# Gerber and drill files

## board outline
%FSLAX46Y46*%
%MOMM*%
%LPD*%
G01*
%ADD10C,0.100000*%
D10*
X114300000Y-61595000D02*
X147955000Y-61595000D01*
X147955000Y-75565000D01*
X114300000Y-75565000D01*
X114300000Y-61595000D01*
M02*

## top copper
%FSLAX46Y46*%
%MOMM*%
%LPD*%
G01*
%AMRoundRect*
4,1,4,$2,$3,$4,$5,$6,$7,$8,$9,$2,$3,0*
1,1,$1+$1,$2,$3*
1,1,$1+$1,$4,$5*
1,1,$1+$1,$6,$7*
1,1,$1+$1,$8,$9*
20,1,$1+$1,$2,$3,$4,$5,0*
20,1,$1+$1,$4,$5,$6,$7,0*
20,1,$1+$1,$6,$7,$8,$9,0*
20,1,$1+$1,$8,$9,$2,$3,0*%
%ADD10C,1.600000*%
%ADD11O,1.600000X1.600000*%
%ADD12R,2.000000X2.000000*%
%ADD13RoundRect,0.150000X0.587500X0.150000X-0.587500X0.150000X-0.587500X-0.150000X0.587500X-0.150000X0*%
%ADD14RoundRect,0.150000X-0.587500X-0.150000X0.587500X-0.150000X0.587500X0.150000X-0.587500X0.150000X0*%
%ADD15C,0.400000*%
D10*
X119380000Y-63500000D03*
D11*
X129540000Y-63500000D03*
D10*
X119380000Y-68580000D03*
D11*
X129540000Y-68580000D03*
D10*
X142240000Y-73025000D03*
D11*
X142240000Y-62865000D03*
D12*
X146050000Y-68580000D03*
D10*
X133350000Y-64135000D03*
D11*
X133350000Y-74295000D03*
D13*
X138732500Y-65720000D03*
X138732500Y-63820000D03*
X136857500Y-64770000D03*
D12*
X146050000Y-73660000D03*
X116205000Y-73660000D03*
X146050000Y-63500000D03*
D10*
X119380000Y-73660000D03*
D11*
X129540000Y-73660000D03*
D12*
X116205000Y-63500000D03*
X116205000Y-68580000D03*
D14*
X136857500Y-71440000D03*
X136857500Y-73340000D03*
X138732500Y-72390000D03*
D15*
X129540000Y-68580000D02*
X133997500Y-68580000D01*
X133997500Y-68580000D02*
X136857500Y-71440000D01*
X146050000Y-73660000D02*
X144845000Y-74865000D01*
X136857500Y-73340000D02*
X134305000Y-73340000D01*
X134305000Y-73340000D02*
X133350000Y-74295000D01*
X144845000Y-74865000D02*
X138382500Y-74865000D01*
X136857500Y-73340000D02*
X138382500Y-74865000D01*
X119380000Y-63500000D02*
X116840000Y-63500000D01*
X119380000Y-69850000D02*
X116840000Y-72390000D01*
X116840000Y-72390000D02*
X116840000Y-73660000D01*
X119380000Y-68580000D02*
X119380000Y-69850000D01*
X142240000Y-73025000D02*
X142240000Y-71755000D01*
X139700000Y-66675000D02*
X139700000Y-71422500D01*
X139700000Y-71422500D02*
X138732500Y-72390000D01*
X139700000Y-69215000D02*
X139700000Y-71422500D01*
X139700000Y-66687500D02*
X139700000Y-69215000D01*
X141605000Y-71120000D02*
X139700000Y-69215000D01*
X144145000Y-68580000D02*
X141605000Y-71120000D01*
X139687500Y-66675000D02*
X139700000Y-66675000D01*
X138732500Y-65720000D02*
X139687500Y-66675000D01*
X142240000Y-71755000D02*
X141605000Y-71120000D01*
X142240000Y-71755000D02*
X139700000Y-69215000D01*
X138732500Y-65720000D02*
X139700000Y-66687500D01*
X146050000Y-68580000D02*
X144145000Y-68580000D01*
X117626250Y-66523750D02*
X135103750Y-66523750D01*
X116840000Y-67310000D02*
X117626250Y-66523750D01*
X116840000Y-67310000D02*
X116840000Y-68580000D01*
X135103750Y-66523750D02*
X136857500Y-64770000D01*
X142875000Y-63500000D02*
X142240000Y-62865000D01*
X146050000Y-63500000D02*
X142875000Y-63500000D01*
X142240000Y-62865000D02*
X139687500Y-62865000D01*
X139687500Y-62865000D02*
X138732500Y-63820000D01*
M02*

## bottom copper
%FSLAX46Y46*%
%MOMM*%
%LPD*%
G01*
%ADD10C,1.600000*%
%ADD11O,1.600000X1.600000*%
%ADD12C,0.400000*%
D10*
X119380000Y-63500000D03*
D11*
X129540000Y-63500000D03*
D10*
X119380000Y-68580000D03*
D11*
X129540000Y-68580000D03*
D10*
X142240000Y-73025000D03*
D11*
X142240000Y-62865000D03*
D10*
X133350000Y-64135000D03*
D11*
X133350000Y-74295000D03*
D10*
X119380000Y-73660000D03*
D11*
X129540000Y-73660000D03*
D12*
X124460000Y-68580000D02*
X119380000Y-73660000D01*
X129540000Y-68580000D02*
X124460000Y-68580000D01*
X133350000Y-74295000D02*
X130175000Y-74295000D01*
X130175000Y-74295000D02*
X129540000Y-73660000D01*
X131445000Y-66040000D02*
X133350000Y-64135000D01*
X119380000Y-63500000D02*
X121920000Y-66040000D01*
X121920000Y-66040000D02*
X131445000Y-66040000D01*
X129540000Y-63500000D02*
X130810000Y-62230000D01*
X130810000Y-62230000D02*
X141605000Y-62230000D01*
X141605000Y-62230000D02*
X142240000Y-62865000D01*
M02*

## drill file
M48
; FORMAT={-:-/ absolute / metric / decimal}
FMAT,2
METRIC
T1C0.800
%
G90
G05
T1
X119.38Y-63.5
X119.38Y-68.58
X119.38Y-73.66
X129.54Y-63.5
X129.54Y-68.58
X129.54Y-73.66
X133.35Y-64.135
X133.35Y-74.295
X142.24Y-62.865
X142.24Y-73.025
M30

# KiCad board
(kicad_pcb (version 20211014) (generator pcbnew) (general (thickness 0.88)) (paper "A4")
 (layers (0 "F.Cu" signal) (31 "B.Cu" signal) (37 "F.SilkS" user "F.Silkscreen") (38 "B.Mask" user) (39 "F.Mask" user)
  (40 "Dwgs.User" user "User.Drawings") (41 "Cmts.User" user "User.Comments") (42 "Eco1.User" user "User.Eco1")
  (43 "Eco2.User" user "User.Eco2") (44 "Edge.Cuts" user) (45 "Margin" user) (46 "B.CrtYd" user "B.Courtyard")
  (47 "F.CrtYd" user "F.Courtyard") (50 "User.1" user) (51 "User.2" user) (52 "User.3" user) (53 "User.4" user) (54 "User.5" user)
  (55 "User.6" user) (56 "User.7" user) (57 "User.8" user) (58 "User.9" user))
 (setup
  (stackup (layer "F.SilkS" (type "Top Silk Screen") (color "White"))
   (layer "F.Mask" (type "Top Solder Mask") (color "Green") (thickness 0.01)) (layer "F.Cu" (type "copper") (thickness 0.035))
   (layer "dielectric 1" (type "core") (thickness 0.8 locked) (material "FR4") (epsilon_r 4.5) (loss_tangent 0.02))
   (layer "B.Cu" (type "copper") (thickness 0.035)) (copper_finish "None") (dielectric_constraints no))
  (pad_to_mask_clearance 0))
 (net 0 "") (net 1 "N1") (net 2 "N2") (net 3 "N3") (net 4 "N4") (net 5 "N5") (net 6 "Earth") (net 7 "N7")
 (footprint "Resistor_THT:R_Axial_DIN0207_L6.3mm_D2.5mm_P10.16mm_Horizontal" (layer "F.Cu") (at 119.38 63.5)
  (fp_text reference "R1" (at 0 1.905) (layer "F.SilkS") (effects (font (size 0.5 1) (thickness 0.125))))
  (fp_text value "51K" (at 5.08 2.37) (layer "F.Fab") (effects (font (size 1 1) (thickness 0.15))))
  (pad "1" thru_hole circle (at 0 0) (size 1.6 1.6) (drill 0.8) (layers *.Cu *.Mask) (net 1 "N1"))
  (pad "2" thru_hole oval (at 10.16 0) (size 1.6 1.6) (drill 0.8) (layers *.Cu *.Mask) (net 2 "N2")))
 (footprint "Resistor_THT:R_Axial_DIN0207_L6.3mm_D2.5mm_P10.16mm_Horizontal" (layer "F.Cu") (at 119.38 68.58)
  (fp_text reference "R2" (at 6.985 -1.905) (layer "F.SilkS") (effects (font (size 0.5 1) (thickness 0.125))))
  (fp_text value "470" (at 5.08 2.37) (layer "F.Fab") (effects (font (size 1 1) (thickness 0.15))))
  (pad "1" thru_hole circle (at 0 0) (size 1.6 1.6) (drill 0.8) (layers *.Cu *.Mask) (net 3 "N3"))
  (pad "2" thru_hole oval (at 10.16 0) (size 1.6 1.6) (drill 0.8) (layers *.Cu *.Mask) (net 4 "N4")))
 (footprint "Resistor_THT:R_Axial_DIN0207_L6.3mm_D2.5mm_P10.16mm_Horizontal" (layer "F.Cu") (at 142.24 73.025 90)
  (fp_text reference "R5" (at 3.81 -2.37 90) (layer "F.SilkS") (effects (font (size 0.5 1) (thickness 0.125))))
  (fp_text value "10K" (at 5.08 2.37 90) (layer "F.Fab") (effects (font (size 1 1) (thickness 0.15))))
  (pad "1" thru_hole circle (at 0 0 90) (size 1.6 1.6) (drill 0.8) (layers *.Cu *.Mask) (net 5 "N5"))
  (pad "2" thru_hole oval (at 10.16 0 90) (size 1.6 1.6) (drill 0.8) (layers *.Cu *.Mask) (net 2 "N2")))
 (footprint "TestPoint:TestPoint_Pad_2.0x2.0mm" (layer "F.Cu") (at 146.05 68.58 90)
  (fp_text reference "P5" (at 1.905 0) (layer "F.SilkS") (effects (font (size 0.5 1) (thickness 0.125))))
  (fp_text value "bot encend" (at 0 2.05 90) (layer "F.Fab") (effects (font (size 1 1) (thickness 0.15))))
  (pad "1" smd rect (at 0 0 90) (size 2 2) (layers "F.Cu" "F.Mask") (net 5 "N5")))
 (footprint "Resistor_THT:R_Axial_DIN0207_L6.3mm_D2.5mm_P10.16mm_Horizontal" (layer "F.Cu") (at 133.35 64.135 -90)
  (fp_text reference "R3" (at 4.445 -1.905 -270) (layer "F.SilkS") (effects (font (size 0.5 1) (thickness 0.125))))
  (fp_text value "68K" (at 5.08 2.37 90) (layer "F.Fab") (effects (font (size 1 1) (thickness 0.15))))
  (pad "1" thru_hole circle (at 0 0 270) (size 1.6 1.6) (drill 0.8) (layers *.Cu *.Mask) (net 1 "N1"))
  (pad "2" thru_hole oval (at 10.16 0 270) (size 1.6 1.6) (drill 0.8) (layers *.Cu *.Mask) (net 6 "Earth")))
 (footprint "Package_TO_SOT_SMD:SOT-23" (layer "F.Cu") (at 137.795 64.77 180)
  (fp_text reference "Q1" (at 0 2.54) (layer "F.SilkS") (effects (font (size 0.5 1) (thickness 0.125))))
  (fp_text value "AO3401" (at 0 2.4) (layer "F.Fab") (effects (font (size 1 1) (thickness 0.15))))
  (pad "1" smd roundrect (at -0.9375 -0.95 180) (size 1.475 0.6) (layers "F.Cu" "F.Paste" "F.Mask") (roundrect_rratio 0.25) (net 5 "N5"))
  (pad "2" smd roundrect (at -0.9375 0.95 180) (size 1.475 0.6) (layers "F.Cu" "F.Paste" "F.Mask") (roundrect_rratio 0.25) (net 2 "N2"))
  (pad "3" smd roundrect (at 0.9375 0 180) (size 1.475 0.6) (layers "F.Cu" "F.Paste" "F.Mask") (roundrect_rratio 0.25) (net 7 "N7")))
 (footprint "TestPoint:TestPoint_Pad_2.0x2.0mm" (layer "F.Cu") (at 146.05 73.66)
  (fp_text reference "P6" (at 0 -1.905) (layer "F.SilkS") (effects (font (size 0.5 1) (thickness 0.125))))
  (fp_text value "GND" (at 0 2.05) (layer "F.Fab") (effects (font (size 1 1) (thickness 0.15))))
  (pad "1" smd rect (at 0 0) (size 2 2) (layers "F.Cu" "F.Mask") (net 6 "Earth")))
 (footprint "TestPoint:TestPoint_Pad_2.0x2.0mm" (layer "F.Cu") (at 116.205 73.66)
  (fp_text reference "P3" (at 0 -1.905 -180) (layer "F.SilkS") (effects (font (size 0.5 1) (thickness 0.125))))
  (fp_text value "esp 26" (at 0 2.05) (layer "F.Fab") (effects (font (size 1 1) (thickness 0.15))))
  (pad "1" smd rect (at 0 0) (size 2 2) (layers "F.Cu" "F.Mask") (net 3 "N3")))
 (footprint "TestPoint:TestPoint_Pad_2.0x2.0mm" (layer "F.Cu") (at 146.05 63.5)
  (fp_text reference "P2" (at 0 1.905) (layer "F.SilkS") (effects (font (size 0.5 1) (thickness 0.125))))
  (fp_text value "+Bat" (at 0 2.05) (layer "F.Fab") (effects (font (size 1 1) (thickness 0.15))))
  (pad "1" smd rect (at 0 0) (size 2 2) (layers "F.Cu" "F.Mask") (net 2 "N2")))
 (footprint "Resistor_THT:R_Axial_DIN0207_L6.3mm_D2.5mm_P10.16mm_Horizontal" (layer "F.Cu") (at 119.38 73.66)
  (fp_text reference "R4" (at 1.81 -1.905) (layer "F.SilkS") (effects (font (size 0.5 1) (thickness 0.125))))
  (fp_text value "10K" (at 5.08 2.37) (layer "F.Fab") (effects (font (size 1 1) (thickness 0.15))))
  (pad "1" thru_hole circle (at 0 0) (size 1.6 1.6) (drill 0.8) (layers *.Cu *.Mask) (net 4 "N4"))
  (pad "2" thru_hole oval (at 10.16 0) (size 1.6 1.6) (drill 0.8) (layers *.Cu *.Mask) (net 6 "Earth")))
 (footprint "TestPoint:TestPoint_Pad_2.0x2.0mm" (layer "F.Cu") (at 116.205 63.5)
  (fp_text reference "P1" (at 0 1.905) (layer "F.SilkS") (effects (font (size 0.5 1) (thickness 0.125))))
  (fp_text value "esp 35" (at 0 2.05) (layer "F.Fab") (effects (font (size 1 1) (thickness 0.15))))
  (pad "1" smd rect (at 0 0) (size 2 2) (layers "F.Cu" "F.Mask") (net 1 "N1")))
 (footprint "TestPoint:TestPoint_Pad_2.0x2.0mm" (layer "F.Cu") (at 116.205 68.58)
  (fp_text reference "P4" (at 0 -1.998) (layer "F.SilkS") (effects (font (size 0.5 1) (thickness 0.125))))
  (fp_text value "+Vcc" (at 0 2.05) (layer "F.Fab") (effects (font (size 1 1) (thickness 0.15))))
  (pad "1" smd rect (at 0 0) (size 2 2) (layers "F.Cu" "F.Mask") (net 7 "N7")))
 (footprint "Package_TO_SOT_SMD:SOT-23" (layer "F.Cu") (at 137.795 72.39)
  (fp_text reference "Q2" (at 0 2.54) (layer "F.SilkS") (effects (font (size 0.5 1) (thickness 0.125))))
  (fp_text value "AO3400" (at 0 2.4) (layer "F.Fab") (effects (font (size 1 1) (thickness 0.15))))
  (pad "1" smd roundrect (at -0.9375 -0.95) (size 1.475 0.6) (layers "F.Cu" "F.Paste" "F.Mask") (roundrect_rratio 0.25) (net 4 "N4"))
  (pad "2" smd roundrect (at -0.9375 0.95) (size 1.475 0.6) (layers "F.Cu" "F.Paste" "F.Mask") (roundrect_rratio 0.25) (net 6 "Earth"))
  (pad "3" smd roundrect (at 0.9375 0) (size 1.475 0.6) (layers "F.Cu" "F.Paste" "F.Mask") (roundrect_rratio 0.25) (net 5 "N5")))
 (gr_rect (start 114.3 61.595) (end 147.955 75.565) (layer "Edge.Cuts") (width 0.1) (fill none))
 (segment (start 129.54 68.58) (end 133.9975 68.58) (width 0.4) (layer "F.Cu") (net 4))
 (segment (start 133.9975 68.58) (end 136.8575 71.44) (width 0.4) (layer "F.Cu") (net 4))
 (segment (start 124.46 68.58) (end 119.38 73.66) (width 0.4) (layer "B.Cu") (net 4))
 (segment (start 129.54 68.58) (end 124.46 68.58) (width 0.4) (layer "B.Cu") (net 4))
 (segment (start 146.05 73.66) (end 144.845 74.865) (width 0.4) (layer "F.Cu") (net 6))
 (segment (start 136.8575 73.34) (end 134.305 73.34) (width 0.4) (layer "F.Cu") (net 6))
 (segment (start 134.305 73.34) (end 133.35 74.295) (width 0.4) (layer "F.Cu") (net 6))
 (segment (start 144.845 74.865) (end 138.3825 74.865) (width 0.4) (layer "F.Cu") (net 6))
 (segment (start 136.8575 73.34) (end 138.3825 74.865) (width 0.4) (layer "F.Cu") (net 6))
 (segment (start 133.35 74.295) (end 130.175 74.295) (width 0.4) (layer "B.Cu") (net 6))
 (segment (start 130.175 74.295) (end 129.54 73.66) (width 0.4) (layer "B.Cu") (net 6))
 (segment (start 119.38 63.5) (end 116.84 63.5) (width 0.4) (layer "F.Cu") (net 1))
 (segment (start 131.445 66.04) (end 133.35 64.135) (width 0.4) (layer "B.Cu") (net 1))
 (segment (start 119.38 63.5) (end 121.92 66.04) (width 0.4) (layer "B.Cu") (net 1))
 (segment (start 121.92 66.04) (end 131.445 66.04) (width 0.4) (layer "B.Cu") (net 1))
 (segment (start 119.38 69.85) (end 116.84 72.39) (width 0.4) (layer "F.Cu") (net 3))
 (segment (start 116.84 72.39) (end 116.84 73.66) (width 0.4) (layer "F.Cu") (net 3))
 (segment (start 119.38 68.58) (end 119.38 69.85) (width 0.4) (layer "F.Cu") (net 3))
 (segment (start 142.24 73.025) (end 142.24 71.755) (width 0.4) (layer "F.Cu") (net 5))
 (segment (start 139.7 66.675) (end 139.7 71.4225) (width 0.4) (layer "F.Cu") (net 5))
 (segment (start 139.7 71.4225) (end 138.7325 72.39) (width 0.4) (layer "F.Cu") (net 5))
 (segment (start 139.7 69.215) (end 139.7 71.4225) (width 0.4) (layer "F.Cu") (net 5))
 (segment (start 139.7 66.6875) (end 139.7 69.215) (width 0.4) (layer "F.Cu") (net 5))
 (segment (start 141.605 71.12) (end 139.7 69.215) (width 0.4) (layer "F.Cu") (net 5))
 (segment (start 144.145 68.58) (end 141.605 71.12) (width 0.4) (layer "F.Cu") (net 5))
 (segment (start 139.6875 66.675) (end 139.7 66.675) (width 0.4) (layer "F.Cu") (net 5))
 (segment (start 138.7325 65.72) (end 139.6875 66.675) (width 0.4) (layer "F.Cu") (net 5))
 (segment (start 142.24 71.755) (end 141.605 71.12) (width 0.4) (layer "F.Cu") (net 5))
 (segment (start 142.24 71.755) (end 139.7 69.215) (width 0.4) (layer "F.Cu") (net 5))
 (segment (start 138.7325 65.72) (end 139.7 66.6875) (width 0.4) (layer "F.Cu") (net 5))
 (segment (start 146.05 68.58) (end 144.145 68.58) (width 0.4) (layer "F.Cu") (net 5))
 (segment (start 117.62625 66.52375) (end 135.10375 66.52375) (width 0.4) (layer "F.Cu") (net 7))
 (segment (start 116.84 67.31) (end 117.62625 66.52375) (width 0.4) (layer "F.Cu") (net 7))
 (segment (start 116.84 67.31) (end 116.84 68.58) (width 0.4) (layer "F.Cu") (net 7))
 (segment (start 135.10375 66.52375) (end 136.8575 64.77) (width 0.4) (layer "F.Cu") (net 7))
 (segment (start 142.875 63.5) (end 142.24 62.865) (width 0.4) (layer "F.Cu") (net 2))
 (segment (start 146.05 63.5) (end 142.875 63.5) (width 0.4) (layer "F.Cu") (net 2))
 (segment (start 142.24 62.865) (end 139.6875 62.865) (width 0.4) (layer "F.Cu") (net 2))
 (segment (start 139.6875 62.865) (end 138.7325 63.82) (width 0.4) (layer "F.Cu") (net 2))
 (segment (start 129.54 63.5) (end 130.81 62.23) (width 0.4) (layer "B.Cu") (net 2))
 (segment (start 130.81 62.23) (end 141.605 62.23) (width 0.4) (layer "B.Cu") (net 2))
 (segment (start 141.605 62.23) (end 142.24 62.865) (width 0.4) (layer "B.Cu") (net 2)))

